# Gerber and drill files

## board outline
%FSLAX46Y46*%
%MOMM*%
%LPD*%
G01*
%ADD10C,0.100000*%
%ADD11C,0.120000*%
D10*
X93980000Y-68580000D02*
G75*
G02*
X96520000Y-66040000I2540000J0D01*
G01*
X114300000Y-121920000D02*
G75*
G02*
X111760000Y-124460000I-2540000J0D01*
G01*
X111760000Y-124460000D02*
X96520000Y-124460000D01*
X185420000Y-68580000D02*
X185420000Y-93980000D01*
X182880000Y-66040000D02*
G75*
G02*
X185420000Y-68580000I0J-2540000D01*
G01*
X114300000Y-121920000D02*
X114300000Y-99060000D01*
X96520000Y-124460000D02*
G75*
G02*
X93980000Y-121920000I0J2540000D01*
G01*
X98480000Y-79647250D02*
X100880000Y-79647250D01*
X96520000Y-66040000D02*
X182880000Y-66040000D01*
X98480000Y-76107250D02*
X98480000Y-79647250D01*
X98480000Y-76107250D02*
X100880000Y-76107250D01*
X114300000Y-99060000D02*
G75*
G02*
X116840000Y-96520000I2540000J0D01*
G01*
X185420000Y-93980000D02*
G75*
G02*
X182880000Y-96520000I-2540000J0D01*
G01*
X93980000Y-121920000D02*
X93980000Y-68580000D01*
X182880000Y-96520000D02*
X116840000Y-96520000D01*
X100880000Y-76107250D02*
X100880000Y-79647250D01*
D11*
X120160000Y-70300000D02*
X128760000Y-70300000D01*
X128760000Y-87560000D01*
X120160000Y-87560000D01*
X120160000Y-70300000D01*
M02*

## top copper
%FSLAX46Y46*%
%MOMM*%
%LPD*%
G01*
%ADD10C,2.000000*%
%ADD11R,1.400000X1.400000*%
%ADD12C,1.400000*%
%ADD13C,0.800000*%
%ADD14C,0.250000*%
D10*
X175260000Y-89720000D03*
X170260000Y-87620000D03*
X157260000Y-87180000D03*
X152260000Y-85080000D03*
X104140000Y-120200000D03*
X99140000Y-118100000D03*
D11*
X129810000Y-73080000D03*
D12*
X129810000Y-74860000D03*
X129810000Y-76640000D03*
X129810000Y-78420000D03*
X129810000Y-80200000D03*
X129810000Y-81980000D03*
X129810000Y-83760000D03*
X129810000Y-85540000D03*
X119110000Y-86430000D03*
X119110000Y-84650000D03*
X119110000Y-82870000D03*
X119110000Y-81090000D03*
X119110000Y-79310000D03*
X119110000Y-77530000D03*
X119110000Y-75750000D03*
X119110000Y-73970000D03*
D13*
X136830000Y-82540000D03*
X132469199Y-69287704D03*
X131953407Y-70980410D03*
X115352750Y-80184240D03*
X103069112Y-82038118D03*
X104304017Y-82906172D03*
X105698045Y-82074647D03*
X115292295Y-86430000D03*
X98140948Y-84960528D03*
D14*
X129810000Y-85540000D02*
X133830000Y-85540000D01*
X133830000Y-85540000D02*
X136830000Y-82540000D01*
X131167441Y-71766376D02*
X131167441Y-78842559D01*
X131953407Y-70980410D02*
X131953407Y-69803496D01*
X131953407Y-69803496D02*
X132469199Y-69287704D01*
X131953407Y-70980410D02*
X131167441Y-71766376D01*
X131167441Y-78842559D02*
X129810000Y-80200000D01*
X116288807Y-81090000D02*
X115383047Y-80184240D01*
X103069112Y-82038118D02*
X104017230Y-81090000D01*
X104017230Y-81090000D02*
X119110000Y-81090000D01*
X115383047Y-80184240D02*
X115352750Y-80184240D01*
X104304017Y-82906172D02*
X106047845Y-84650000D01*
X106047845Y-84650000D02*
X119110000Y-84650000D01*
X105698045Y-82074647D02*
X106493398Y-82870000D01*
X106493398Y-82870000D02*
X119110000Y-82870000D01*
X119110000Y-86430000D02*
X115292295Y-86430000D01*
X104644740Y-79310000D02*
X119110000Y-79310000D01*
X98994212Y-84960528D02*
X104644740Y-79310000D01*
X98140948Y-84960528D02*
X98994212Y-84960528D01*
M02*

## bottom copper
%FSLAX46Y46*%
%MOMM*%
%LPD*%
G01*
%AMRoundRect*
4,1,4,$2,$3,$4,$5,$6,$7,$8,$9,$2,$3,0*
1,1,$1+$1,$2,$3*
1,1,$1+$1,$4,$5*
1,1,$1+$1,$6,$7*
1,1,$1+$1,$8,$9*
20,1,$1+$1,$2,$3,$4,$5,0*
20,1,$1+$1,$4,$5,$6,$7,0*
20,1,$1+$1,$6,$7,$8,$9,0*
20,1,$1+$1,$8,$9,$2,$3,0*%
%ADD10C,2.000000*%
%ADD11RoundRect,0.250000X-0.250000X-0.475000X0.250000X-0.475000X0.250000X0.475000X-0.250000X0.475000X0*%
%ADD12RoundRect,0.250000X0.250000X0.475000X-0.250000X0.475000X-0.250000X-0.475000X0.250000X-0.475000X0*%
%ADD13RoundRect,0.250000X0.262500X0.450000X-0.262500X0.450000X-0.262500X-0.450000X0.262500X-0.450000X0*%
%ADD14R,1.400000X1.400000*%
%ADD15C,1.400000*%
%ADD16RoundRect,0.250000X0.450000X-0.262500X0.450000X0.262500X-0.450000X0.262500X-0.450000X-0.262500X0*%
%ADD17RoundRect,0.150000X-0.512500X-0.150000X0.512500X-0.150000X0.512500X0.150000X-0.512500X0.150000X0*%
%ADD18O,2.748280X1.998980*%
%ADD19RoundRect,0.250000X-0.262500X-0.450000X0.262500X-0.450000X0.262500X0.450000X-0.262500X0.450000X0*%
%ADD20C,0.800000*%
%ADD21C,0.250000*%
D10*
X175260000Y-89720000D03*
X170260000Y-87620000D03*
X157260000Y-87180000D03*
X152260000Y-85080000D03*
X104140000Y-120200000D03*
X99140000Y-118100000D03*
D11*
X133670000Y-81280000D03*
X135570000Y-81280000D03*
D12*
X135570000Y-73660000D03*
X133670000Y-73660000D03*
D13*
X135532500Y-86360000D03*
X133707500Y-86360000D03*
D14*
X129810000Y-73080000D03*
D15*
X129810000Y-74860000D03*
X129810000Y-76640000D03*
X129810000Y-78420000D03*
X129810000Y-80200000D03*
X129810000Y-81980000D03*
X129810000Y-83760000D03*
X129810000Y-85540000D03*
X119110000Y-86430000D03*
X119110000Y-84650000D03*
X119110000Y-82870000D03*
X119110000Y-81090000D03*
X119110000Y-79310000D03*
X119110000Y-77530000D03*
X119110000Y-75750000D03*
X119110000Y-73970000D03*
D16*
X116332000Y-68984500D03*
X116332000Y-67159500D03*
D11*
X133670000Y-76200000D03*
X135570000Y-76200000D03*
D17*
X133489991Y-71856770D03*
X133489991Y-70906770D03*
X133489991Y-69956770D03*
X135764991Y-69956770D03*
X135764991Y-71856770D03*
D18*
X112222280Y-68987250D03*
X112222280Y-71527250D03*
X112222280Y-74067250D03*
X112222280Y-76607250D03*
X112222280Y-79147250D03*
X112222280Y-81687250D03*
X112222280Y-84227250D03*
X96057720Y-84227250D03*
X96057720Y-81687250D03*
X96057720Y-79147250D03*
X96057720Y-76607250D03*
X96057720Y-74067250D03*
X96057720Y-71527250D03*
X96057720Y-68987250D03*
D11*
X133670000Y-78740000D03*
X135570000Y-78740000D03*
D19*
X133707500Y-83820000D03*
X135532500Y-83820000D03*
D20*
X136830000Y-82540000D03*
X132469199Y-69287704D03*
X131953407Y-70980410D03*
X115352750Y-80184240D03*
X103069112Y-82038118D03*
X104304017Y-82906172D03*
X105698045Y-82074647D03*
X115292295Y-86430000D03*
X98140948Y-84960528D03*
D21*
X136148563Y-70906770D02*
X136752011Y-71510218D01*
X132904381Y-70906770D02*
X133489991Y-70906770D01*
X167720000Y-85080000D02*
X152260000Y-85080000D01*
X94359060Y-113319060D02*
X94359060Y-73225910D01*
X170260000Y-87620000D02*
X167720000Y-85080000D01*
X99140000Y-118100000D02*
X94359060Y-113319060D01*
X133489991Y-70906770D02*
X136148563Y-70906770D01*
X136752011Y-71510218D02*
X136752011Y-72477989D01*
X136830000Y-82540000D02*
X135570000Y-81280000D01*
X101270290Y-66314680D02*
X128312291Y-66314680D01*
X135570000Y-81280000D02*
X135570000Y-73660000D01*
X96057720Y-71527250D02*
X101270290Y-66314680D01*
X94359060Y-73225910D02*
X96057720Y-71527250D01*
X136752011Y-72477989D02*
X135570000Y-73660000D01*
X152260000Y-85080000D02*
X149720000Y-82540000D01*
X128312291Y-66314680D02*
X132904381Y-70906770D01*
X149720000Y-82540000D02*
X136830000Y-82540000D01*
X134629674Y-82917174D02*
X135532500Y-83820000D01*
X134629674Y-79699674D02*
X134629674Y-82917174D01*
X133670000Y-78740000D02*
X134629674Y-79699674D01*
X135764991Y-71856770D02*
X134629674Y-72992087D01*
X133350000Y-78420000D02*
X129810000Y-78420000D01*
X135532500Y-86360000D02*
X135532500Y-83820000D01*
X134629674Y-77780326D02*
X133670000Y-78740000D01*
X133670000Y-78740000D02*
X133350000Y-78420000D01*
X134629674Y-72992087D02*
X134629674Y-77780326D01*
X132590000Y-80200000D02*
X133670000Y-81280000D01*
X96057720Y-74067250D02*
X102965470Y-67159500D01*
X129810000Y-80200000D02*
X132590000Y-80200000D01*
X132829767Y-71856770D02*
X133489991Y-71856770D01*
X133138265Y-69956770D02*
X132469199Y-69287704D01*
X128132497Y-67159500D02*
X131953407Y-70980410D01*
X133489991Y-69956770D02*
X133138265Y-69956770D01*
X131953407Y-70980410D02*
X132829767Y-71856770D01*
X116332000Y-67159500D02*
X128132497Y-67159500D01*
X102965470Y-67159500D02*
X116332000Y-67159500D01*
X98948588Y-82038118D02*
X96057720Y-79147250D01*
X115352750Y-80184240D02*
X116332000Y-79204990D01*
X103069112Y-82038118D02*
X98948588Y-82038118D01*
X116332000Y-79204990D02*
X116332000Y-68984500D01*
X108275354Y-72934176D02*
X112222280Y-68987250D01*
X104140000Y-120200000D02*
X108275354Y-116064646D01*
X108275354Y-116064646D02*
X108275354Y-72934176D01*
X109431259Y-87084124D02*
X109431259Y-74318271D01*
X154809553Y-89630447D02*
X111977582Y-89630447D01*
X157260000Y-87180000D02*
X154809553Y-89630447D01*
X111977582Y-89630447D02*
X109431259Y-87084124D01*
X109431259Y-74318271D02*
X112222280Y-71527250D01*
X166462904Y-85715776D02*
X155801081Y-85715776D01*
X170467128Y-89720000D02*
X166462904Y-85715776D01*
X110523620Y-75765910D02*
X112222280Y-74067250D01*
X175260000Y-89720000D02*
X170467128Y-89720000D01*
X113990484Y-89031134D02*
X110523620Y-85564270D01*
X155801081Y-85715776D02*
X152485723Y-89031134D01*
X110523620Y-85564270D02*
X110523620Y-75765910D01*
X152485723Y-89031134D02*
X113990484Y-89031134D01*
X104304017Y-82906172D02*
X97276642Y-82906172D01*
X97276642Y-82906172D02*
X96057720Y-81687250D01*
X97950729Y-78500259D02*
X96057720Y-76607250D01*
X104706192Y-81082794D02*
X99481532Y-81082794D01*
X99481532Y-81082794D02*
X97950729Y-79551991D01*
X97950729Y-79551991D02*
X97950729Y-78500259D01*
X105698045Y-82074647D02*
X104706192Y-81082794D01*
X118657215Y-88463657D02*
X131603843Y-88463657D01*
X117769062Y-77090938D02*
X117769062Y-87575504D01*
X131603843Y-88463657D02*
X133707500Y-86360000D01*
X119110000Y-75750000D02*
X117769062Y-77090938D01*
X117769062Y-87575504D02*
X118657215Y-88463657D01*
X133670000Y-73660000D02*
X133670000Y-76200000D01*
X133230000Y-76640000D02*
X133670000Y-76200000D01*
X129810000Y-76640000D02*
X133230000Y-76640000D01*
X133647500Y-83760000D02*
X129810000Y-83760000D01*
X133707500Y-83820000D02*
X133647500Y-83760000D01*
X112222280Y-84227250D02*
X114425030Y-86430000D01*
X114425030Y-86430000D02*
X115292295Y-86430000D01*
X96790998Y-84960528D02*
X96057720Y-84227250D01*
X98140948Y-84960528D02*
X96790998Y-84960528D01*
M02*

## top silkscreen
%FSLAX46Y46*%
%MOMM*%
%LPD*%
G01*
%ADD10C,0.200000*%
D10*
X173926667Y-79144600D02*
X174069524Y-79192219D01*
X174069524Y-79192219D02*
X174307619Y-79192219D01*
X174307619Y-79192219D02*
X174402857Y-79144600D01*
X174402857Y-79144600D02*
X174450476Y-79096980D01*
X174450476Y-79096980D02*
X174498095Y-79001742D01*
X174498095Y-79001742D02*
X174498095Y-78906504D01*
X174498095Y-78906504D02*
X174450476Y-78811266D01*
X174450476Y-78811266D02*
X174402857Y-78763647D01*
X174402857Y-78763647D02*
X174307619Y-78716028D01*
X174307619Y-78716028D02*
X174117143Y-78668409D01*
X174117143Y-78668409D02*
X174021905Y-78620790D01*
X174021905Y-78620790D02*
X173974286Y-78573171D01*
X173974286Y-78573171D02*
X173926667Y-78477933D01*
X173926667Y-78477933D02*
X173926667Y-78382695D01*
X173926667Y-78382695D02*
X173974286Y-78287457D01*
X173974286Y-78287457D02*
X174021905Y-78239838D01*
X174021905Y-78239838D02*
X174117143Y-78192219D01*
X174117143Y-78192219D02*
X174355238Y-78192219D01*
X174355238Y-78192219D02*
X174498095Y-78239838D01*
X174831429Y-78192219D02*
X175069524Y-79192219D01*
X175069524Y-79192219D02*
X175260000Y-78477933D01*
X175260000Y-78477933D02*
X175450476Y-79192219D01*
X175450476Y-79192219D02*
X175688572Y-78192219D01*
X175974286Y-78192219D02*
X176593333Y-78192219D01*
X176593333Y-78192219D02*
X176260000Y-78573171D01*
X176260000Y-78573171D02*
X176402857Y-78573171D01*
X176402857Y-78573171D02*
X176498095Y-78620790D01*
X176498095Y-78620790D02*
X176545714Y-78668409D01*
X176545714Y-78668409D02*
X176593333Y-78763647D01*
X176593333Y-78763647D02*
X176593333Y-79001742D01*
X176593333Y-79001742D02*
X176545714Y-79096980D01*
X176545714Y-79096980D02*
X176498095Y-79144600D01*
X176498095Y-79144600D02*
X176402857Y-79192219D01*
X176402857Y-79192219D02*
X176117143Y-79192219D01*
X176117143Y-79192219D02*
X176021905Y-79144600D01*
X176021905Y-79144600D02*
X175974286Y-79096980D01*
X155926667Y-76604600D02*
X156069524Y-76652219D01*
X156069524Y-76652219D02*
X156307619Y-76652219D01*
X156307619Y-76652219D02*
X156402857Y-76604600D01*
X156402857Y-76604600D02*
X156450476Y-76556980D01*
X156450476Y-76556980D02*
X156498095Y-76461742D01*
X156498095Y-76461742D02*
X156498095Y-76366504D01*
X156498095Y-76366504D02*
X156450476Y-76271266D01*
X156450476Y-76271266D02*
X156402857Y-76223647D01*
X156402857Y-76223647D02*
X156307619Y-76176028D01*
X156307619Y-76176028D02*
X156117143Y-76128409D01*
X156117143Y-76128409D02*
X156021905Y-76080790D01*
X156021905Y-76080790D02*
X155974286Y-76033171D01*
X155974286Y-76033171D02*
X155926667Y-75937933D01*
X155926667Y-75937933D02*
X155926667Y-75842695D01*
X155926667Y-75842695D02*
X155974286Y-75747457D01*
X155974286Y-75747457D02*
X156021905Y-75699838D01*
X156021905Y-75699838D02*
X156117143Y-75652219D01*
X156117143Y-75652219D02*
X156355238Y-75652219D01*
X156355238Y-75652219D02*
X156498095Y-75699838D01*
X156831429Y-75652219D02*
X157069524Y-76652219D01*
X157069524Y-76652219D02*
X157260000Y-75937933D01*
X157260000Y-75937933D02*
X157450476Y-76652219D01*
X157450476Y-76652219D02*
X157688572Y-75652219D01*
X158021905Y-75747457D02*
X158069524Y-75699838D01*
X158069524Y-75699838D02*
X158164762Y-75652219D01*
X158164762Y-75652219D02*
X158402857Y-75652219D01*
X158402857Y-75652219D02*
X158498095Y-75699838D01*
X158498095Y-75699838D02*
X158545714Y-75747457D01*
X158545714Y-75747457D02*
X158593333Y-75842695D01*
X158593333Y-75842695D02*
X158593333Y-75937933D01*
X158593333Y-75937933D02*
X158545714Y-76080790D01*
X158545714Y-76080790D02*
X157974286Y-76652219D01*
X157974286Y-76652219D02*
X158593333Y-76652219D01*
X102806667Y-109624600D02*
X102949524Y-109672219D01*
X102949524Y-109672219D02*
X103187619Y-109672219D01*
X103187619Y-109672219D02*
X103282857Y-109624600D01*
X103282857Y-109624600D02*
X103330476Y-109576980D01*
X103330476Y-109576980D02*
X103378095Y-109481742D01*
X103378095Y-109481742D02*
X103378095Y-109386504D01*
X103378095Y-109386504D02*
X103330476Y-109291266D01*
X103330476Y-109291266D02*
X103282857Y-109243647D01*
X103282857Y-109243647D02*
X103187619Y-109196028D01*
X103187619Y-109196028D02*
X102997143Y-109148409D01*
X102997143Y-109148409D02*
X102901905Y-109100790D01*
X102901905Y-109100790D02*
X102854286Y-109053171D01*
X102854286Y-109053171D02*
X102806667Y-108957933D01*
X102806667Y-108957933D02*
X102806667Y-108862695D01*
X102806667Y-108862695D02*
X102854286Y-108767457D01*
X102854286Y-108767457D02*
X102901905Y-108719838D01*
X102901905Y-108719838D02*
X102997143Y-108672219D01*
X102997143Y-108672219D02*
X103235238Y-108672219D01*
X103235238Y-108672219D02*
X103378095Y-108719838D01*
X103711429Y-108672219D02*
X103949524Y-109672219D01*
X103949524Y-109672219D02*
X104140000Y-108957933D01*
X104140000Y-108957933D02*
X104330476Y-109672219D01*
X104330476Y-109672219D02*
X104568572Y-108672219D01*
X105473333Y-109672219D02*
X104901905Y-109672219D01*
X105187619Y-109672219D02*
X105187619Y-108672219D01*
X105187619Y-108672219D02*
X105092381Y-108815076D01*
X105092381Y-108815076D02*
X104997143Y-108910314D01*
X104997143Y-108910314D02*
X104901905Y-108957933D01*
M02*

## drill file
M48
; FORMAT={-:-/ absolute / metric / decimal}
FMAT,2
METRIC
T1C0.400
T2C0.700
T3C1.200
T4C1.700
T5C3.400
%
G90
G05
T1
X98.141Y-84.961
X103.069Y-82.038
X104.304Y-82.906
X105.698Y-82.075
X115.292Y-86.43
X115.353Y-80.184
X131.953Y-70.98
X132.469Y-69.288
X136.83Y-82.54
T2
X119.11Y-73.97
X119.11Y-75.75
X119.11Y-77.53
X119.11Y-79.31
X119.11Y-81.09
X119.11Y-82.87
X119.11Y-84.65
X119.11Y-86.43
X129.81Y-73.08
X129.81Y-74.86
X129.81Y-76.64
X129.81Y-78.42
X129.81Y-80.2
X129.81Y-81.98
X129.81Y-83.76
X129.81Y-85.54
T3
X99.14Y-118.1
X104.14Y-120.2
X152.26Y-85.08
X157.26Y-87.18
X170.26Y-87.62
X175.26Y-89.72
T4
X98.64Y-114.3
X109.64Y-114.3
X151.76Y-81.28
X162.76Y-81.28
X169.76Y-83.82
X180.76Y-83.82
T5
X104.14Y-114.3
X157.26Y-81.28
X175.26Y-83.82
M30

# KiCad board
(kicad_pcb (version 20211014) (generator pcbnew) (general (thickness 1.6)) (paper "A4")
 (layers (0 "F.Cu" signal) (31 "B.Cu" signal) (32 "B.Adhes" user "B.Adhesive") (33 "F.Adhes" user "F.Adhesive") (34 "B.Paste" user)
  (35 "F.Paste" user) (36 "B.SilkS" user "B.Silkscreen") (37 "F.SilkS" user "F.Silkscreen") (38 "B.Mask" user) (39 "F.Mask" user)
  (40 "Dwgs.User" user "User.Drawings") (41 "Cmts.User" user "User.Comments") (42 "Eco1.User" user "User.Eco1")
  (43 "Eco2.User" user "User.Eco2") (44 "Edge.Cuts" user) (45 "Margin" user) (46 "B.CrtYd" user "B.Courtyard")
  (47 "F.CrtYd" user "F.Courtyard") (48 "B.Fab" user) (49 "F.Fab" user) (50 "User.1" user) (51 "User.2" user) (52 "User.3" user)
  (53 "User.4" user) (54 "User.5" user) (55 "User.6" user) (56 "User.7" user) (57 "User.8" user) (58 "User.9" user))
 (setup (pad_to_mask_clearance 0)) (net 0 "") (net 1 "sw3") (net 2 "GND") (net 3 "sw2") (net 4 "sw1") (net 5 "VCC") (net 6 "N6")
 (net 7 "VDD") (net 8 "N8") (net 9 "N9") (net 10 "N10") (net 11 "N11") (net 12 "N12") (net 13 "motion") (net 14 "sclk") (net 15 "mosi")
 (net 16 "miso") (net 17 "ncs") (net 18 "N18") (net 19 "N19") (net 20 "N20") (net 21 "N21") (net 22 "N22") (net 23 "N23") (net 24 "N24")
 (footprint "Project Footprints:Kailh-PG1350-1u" (layer "F.Cu") (at 175.26 83.82)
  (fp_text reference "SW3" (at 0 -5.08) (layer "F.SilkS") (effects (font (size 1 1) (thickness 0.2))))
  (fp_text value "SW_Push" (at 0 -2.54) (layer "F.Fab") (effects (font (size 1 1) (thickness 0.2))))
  (pad "" np_thru_hole circle (at 0 0 180) (size 3.4 3.4) (drill 3.4) (layers *.Cu *.Mask))
  (pad "" np_thru_hole circle (at -5.5 0 180) (size 1.7 1.7) (drill 1.7) (layers *.Cu *.Mask))
  (pad "" np_thru_hole circle (at 5.5 0 180) (size 1.7 1.7) (drill 1.7) (layers *.Cu *.Mask))
  (pad "1" thru_hole circle (at 0 5.9 180) (size 2 2) (drill 1.2) (layers *.Cu *.Mask) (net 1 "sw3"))
  (pad "2" thru_hole circle (at -5 3.8 41.9) (size 2 2) (drill 1.2) (layers *.Cu *.Mask) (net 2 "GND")))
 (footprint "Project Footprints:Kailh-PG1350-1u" (layer "F.Cu") (at 157.26 81.28)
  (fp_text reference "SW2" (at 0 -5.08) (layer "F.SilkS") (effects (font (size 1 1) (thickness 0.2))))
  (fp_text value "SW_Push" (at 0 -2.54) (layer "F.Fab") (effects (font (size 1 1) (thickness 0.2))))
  (pad "" np_thru_hole circle (at 5.5 0 180) (size 1.7 1.7) (drill 1.7) (layers *.Cu *.Mask))
  (pad "" np_thru_hole circle (at -5.5 0 180) (size 1.7 1.7) (drill 1.7) (layers *.Cu *.Mask))
  (pad "" np_thru_hole circle (at 0 0 180) (size 3.4 3.4) (drill 3.4) (layers *.Cu *.Mask))
  (pad "1" thru_hole circle (at 0 5.9 180) (size 2 2) (drill 1.2) (layers *.Cu *.Mask) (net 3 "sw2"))
  (pad "2" thru_hole circle (at -5 3.8 41.9) (size 2 2) (drill 1.2) (layers *.Cu *.Mask) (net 2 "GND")))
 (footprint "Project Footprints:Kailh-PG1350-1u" (layer "F.Cu") (at 104.14 114.3)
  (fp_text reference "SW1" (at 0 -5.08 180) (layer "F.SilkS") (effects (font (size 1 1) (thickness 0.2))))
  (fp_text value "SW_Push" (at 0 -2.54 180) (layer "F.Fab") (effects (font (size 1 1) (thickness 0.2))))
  (pad "" np_thru_hole circle (at 0 0 180) (size 3.4 3.4) (drill 3.4) (layers *.Cu *.Mask))
  (pad "" np_thru_hole circle (at 5.5 0 180) (size 1.7 1.7) (drill 1.7) (layers *.Cu *.Mask))
  (pad "" np_thru_hole circle (at -5.5 0 180) (size 1.7 1.7) (drill 1.7) (layers *.Cu *.Mask))
  (pad "1" thru_hole circle (at 0 5.9 180) (size 2 2) (drill 1.2) (layers *.Cu *.Mask) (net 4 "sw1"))
  (pad "2" thru_hole circle (at -5 3.8 41.9) (size 2 2) (drill 1.2) (layers *.Cu *.Mask) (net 2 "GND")))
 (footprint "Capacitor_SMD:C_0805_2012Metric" (layer "B.Cu") (at 134.62 81.28)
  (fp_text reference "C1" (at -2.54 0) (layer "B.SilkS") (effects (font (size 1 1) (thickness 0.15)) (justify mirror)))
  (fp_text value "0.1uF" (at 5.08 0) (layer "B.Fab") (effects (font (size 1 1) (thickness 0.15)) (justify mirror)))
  (pad "1" smd roundrect (at -0.95 0) (size 1 1.45) (layers "B.Cu" "B.Paste" "B.Mask") (roundrect_rratio 0.25) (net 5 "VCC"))
  (pad "2" smd roundrect (at 0.95 0) (size 1 1.45) (layers "B.Cu" "B.Paste" "B.Mask") (roundrect_rratio 0.25) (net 2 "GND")))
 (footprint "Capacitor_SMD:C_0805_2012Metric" (layer "B.Cu") (at 134.62 73.66 180)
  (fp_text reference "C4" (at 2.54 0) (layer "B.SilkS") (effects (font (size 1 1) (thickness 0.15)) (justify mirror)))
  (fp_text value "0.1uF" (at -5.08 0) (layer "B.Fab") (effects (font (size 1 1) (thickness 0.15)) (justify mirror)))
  (pad "1" smd roundrect (at -0.95 0 180) (size 1 1.45) (layers "B.Cu" "B.Paste" "B.Mask") (roundrect_rratio 0.25) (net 2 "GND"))
  (pad "2" smd roundrect (at 0.95 0 180) (size 1 1.45) (layers "B.Cu" "B.Paste" "B.Mask") (roundrect_rratio 0.25) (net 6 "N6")))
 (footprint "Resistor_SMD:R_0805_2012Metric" (layer "B.Cu") (at 134.62 86.36 180)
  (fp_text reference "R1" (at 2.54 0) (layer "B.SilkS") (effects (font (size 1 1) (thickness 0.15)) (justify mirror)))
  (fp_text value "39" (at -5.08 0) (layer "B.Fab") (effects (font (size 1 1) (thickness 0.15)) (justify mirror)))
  (pad "1" smd roundrect (at -0.9125 0 180) (size 1.025 1.4) (layers "B.Cu" "B.Paste" "B.Mask") (roundrect_rratio 0.243902) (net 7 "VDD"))
  (pad "2" smd roundrect (at 0.9125 0 180) (size 1.025 1.4) (layers "B.Cu" "B.Paste" "B.Mask") (roundrect_rratio 0.243902) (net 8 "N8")))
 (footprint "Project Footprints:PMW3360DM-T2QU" (layer "B.Cu") (at 124.46 78.74 -90)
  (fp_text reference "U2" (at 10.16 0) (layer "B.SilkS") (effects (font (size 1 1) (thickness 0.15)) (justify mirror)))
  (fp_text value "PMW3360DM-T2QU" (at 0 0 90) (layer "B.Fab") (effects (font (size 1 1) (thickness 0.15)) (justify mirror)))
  (fp_rect (start -8.44 4.3) (end 8.82 -4.3) (layer "Edge.Cuts") (width 0.12) (fill none))
  (pad "1" thru_hole rect (at -5.66 -5.35 270) (size 1.4 1.4) (drill 0.7) (layers *.Cu *.Mask) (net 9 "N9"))
  (pad "2" thru_hole circle (at -3.88 -5.35 270) (size 1.4 1.4) (drill 0.7) (layers *.Cu *.Mask) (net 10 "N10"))
  (pad "3" thru_hole circle (at -2.1 -5.35 270) (size 1.4 1.4) (drill 0.7) (layers *.Cu *.Mask) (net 6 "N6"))
  (pad "4" thru_hole circle (at -0.32 -5.35 270) (size 1.4 1.4) (drill 0.7) (layers *.Cu *.Mask) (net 7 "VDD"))
  (pad "5" thru_hole circle (at 1.46 -5.35 270) (size 1.4 1.4) (drill 0.7) (layers *.Cu *.Mask) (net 5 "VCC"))
  (pad "6" thru_hole circle (at 3.24 -5.35 270) (size 1.4 1.4) (drill 0.7) (layers *.Cu *.Mask) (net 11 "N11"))
  (pad "7" thru_hole circle (at 5.02 -5.35 270) (size 1.4 1.4) (drill 0.7) (layers *.Cu *.Mask) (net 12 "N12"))
  (pad "8" thru_hole circle (at 6.8 -5.35 270) (size 1.4 1.4) (drill 0.7) (layers *.Cu *.Mask) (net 2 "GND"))
  (pad "9" thru_hole circle (at 7.69 5.35 270) (size 1.4 1.4) (drill 0.7) (layers *.Cu *.Mask) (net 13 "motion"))
  (pad "10" thru_hole circle (at 5.91 5.35 270) (size 1.4 1.4) (drill 0.7) (layers *.Cu *.Mask) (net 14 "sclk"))
  (pad "11" thru_hole circle (at 4.13 5.35 270) (size 1.4 1.4) (drill 0.7) (layers *.Cu *.Mask) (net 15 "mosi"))
  (pad "12" thru_hole circle (at 2.35 5.35 270) (size 1.4 1.4) (drill 0.7) (layers *.Cu *.Mask) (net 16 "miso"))
  (pad "13" thru_hole circle (at 0.57 5.35 270) (size 1.4 1.4) (drill 0.7) (layers *.Cu *.Mask) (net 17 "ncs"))
  (pad "14" thru_hole circle (at -1.21 5.35 270) (size 1.4 1.4) (drill 0.7) (layers *.Cu *.Mask) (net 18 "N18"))
  (pad "15" thru_hole circle (at -2.99 5.35 270) (size 1.4 1.4) (drill 0.7) (layers *.Cu *.Mask) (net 8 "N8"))
  (pad "16" thru_hole circle (at -4.77 5.35 270) (size 1.4 1.4) (drill 0.7) (layers *.Cu *.Mask) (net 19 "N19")))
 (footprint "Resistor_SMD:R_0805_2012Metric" (layer "B.Cu") (at 116.332 68.072 90)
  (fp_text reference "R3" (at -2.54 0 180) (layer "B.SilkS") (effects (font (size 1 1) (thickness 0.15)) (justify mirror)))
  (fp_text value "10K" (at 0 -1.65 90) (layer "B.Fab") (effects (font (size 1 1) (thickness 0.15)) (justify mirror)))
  (pad "1" smd roundrect (at -0.9125 0 90) (size 1.025 1.4) (layers "B.Cu" "B.Paste" "B.Mask") (roundrect_rratio 0.243902) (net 16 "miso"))
  (pad "2" smd roundrect (at 0.9125 0 90) (size 1.025 1.4) (layers "B.Cu" "B.Paste" "B.Mask") (roundrect_rratio 0.243902) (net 5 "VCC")))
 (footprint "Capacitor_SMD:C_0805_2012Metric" (layer "B.Cu") (at 134.62 76.2)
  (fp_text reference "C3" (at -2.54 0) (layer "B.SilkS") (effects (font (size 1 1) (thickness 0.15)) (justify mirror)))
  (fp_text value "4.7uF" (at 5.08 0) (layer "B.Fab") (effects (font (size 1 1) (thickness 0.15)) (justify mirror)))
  (pad "1" smd roundrect (at -0.95 0) (size 1 1.45) (layers "B.Cu" "B.Paste" "B.Mask") (roundrect_rratio 0.25) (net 6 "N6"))
  (pad "2" smd roundrect (at 0.95 0) (size 1 1.45) (layers "B.Cu" "B.Paste" "B.Mask") (roundrect_rratio 0.25) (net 2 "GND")))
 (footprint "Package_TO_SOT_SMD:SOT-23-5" (layer "B.Cu") (at 134.627491 70.90677)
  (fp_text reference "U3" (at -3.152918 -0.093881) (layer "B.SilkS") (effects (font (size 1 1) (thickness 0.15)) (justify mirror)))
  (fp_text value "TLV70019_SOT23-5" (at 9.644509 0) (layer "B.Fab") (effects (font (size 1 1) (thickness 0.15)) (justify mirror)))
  (pad "1" smd roundrect (at -1.1375 0.95) (size 1.325 0.6) (layers "B.Cu" "B.Paste" "B.Mask") (roundrect_rratio 0.25) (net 5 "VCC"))
  (pad "2" smd roundrect (at -1.1375 0) (size 1.325 0.6) (layers "B.Cu" "B.Paste" "B.Mask") (roundrect_rratio 0.25) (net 2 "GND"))
  (pad "3" smd roundrect (at -1.1375 -0.95) (size 1.325 0.6) (layers "B.Cu" "B.Paste" "B.Mask") (roundrect_rratio 0.25) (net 5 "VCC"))
  (pad "4" smd roundrect (at 1.1375 -0.95) (size 1.325 0.6) (layers "B.Cu" "B.Paste" "B.Mask") (roundrect_rratio 0.25) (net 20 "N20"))
  (pad "5" smd roundrect (at 1.1375 0.95) (size 1.325 0.6) (layers "B.Cu" "B.Paste" "B.Mask") (roundrect_rratio 0.25) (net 7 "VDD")))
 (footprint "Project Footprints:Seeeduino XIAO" (layer "B.Cu") (at 104.14 76.60725 180)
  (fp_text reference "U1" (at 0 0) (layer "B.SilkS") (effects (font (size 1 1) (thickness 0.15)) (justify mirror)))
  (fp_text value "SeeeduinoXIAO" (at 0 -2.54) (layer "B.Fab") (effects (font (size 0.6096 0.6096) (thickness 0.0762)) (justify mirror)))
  (pad "1" smd oval (at -8.08228 7.62 180) (size 2.74828 1.99898) (layers "B.Cu" "B.Paste" "B.Mask") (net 4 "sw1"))
  (pad "2" smd oval (at -8.08228 5.08 180) (size 2.74828 1.99898) (layers "B.Cu" "B.Paste" "B.Mask") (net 3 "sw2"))
  (pad "3" smd oval (at -8.08228 2.54 180) (size 2.74828 1.99898) (layers "B.Cu" "B.Paste" "B.Mask") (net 1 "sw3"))
  (pad "4" smd oval (at -8.08228 0 180) (size 2.74828 1.99898) (layers "B.Cu" "B.Paste" "B.Mask") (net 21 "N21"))
  (pad "5" smd oval (at -8.08228 -2.54 180) (size 2.74828 1.99898) (layers "B.Cu" "B.Paste" "B.Mask") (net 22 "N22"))
  (pad "6" smd oval (at -8.08228 -5.08 180) (size 2.74828 1.99898) (layers "B.Cu" "B.Paste" "B.Mask") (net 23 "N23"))
  (pad "7" smd oval (at -8.08228 -7.62 180) (size 2.74828 1.99898) (layers "B.Cu" "B.Paste" "B.Mask") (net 13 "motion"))
  (pad "8" smd oval (at 8.08228 -7.62 180) (size 2.74828 1.99898) (layers "B.Cu" "B.Paste" "B.Mask") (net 17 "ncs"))
  (pad "9" smd oval (at 8.08228 -5.08 180) (size 2.74828 1.99898) (layers "B.Cu" "B.Paste" "B.Mask") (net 14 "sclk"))
  (pad "10" smd oval (at 8.08228 -2.54 180) (size 2.74828 1.99898) (layers "B.Cu" "B.Paste" "B.Mask") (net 16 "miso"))
  (pad "11" smd oval (at 8.08228 0 180) (size 2.74828 1.99898) (layers "B.Cu" "B.Paste" "B.Mask") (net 15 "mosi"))
  (pad "12" smd oval (at 8.08228 2.54 180) (size 2.74828 1.99898) (layers "B.Cu" "B.Paste" "B.Mask") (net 5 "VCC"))
  (pad "13" smd oval (at 8.08228 5.08 180) (size 2.74828 1.99898) (layers "B.Cu" "B.Paste" "B.Mask") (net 2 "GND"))
  (pad "14" smd oval (at 8.08228 7.62 180) (size 2.74828 1.99898) (layers "B.Cu" "B.Paste" "B.Mask") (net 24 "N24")))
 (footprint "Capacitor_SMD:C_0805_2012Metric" (layer "B.Cu") (at 134.62 78.74)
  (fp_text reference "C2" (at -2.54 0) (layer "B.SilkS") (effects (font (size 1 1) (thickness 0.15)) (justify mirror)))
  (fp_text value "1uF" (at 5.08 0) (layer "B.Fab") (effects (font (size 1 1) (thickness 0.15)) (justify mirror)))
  (pad "1" smd roundrect (at -0.95 0) (size 1 1.45) (layers "B.Cu" "B.Paste" "B.Mask") (roundrect_rratio 0.25) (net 7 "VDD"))
  (pad "2" smd roundrect (at 0.95 0) (size 1 1.45) (layers "B.Cu" "B.Paste" "B.Mask") (roundrect_rratio 0.25) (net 2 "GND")))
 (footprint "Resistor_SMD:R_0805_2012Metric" (layer "B.Cu") (at 134.62 83.82)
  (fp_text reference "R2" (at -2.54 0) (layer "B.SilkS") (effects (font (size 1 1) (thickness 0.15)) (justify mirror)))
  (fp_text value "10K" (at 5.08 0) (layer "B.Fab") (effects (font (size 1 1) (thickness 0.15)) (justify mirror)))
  (pad "1" smd roundrect (at -0.9125 0) (size 1.025 1.4) (layers "B.Cu" "B.Paste" "B.Mask") (roundrect_rratio 0.243902) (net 12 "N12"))
  (pad "2" smd roundrect (at 0.9125 0) (size 1.025 1.4) (layers "B.Cu" "B.Paste" "B.Mask") (roundrect_rratio 0.243902) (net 7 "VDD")))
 (gr_arc (start 93.98 68.58) (mid 94.723949 66.783949) (end 96.52 66.04) (layer "Edge.Cuts") (width 0.1))
 (gr_arc (start 114.3 121.92) (mid 113.556051 123.716051) (end 111.76 124.46) (layer "Edge.Cuts") (width 0.1))
 (gr_line (start 111.76 124.46) (end 96.52 124.46) (layer "Edge.Cuts") (width 0.1))
 (gr_line (start 185.42 68.58) (end 185.42 93.98) (layer "Edge.Cuts") (width 0.1))
 (gr_arc (start 182.88 66.04) (mid 184.676051 66.783949) (end 185.42 68.58) (layer "Edge.Cuts") (width 0.1))
 (gr_line (start 114.3 121.92) (end 114.3 99.06) (layer "Edge.Cuts") (width 0.1))
 (gr_arc (start 96.52 124.46) (mid 94.723949 123.716051) (end 93.98 121.92) (layer "Edge.Cuts") (width 0.1))
 (gr_line (start 98.48 79.64725) (end 100.88 79.64725) (layer "Edge.Cuts") (width 0.1))
 (gr_line (start 96.52 66.04) (end 182.88 66.04) (layer "Edge.Cuts") (width 0.1))
 (gr_line (start 98.48 76.10725) (end 98.48 79.64725) (layer "Edge.Cuts") (width 0.1))
 (gr_line (start 98.48 76.10725) (end 100.88 76.10725) (layer "Edge.Cuts") (width 0.1))
 (gr_arc (start 114.3 99.06) (mid 115.043949 97.263949) (end 116.84 96.52) (layer "Edge.Cuts") (width 0.1))
 (gr_arc (start 185.42 93.98) (mid 184.676051 95.776051) (end 182.88 96.52) (layer "Edge.Cuts") (width 0.1))
 (gr_line (start 93.98 121.92) (end 93.98 68.58) (layer "Edge.Cuts") (width 0.1))
 (gr_line (start 182.88 96.52) (end 116.84 96.52) (layer "Edge.Cuts") (width 0.1))
 (gr_line (start 100.88 76.10725) (end 100.88 79.64725) (layer "Edge.Cuts") (width 0.1))
 (segment (start 129.81 85.54) (end 133.83 85.54) (width 0.25) (layer "F.Cu") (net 2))
 (segment (start 133.83 85.54) (end 136.83 82.54) (width 0.25) (layer "F.Cu") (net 2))
 (via (at 136.83 82.54) (size 0.8) (drill 0.4) (layers "F.Cu" "B.Cu") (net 2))
 (segment (start 136.148563 70.90677) (end 136.752011 71.510218) (width 0.25) (layer "B.Cu") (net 2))
 (segment (start 132.904381 70.90677) (end 133.489991 70.90677) (width 0.25) (layer "B.Cu") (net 2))
 (segment (start 167.72 85.08) (end 152.26 85.08) (width 0.25) (layer "B.Cu") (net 2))
 (segment (start 94.35906 113.31906) (end 94.35906 73.22591) (width 0.25) (layer "B.Cu") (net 2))
 (segment (start 170.26 87.62) (end 167.72 85.08) (width 0.25) (layer "B.Cu") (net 2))
 (segment (start 99.14 118.1) (end 94.35906 113.31906) (width 0.25) (layer "B.Cu") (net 2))
 (segment (start 133.489991 70.90677) (end 136.148563 70.90677) (width 0.25) (layer "B.Cu") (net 2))
 (segment (start 136.752011 71.510218) (end 136.752011 72.477989) (width 0.25) (layer "B.Cu") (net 2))
 (segment (start 136.83 82.54) (end 135.57 81.28) (width 0.25) (layer "B.Cu") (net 2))
 (segment (start 101.27029 66.31468) (end 128.312291 66.31468) (width 0.25) (layer "B.Cu") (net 2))
 (segment (start 135.57 81.28) (end 135.57 73.66) (width 0.25) (layer "B.Cu") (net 2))
 (segment (start 96.05772 71.52725) (end 101.27029 66.31468) (width 0.25) (layer "B.Cu") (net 2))
 (segment (start 94.35906 73.22591) (end 96.05772 71.52725) (width 0.25) (layer "B.Cu") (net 2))
 (segment (start 136.752011 72.477989) (end 135.57 73.66) (width 0.25) (layer "B.Cu") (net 2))
 (segment (start 152.26 85.08) (end 149.72 82.54) (width 0.25) (layer "B.Cu") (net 2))
 (segment (start 128.312291 66.31468) (end 132.904381 70.90677) (width 0.25) (layer "B.Cu") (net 2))
 (segment (start 149.72 82.54) (end 136.83 82.54) (width 0.25) (layer "B.Cu") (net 2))
 (segment (start 134.629674 82.917174) (end 135.5325 83.82) (width 0.25) (layer "B.Cu") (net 7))
 (segment (start 134.629674 79.699674) (end 134.629674 82.917174) (width 0.25) (layer "B.Cu") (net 7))
 (segment (start 133.67 78.74) (end 134.629674 79.699674) (width 0.25) (layer "B.Cu") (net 7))
 (segment (start 135.764991 71.85677) (end 134.629674 72.992087) (width 0.25) (layer "B.Cu") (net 7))
 (segment (start 133.35 78.42) (end 129.81 78.42) (width 0.25) (layer "B.Cu") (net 7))
 (segment (start 135.5325 86.36) (end 135.5325 83.82) (width 0.25) (layer "B.Cu") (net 7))
 (segment (start 134.629674 77.780326) (end 133.67 78.74) (width 0.25) (layer "B.Cu") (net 7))
 (segment (start 133.67 78.74) (end 133.35 78.42) (width 0.25) (layer "B.Cu") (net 7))
 (segment (start 134.629674 72.992087) (end 134.629674 77.780326) (width 0.25) (layer "B.Cu") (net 7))
 (segment (start 131.167441 71.766376) (end 131.167441 78.842559) (width 0.25) (layer "F.Cu") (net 5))
 (segment (start 131.953407 70.98041) (end 131.953407 69.803496) (width 0.25) (layer "F.Cu") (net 5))
 (segment (start 131.953407 69.803496) (end 132.469199 69.287704) (width 0.25) (layer "F.Cu") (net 5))
 (segment (start 131.953407 70.98041) (end 131.167441 71.766376) (width 0.25) (layer "F.Cu") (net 5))
 (segment (start 131.167441 78.842559) (end 129.81 80.2) (width 0.25) (layer "F.Cu") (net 5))
 (via (at 132.469199 69.287704) (size 0.8) (drill 0.4) (layers "F.Cu" "B.Cu") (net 5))
 (via (at 131.953407 70.98041) (size 0.8) (drill 0.4) (layers "F.Cu" "B.Cu") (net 5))
 (segment (start 132.59 80.2) (end 133.67 81.28) (width 0.25) (layer "B.Cu") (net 5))
 (segment (start 96.05772 74.06725) (end 102.96547 67.1595) (width 0.25) (layer "B.Cu") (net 5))
 (segment (start 129.81 80.2) (end 132.59 80.2) (width 0.25) (layer "B.Cu") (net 5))
 (segment (start 132.829767 71.85677) (end 133.489991 71.85677) (width 0.25) (layer "B.Cu") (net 5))
 (segment (start 133.138265 69.95677) (end 132.469199 69.287704) (width 0.25) (layer "B.Cu") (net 5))
 (segment (start 128.132497 67.1595) (end 131.953407 70.98041) (width 0.25) (layer "B.Cu") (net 5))
 (segment (start 133.489991 69.95677) (end 133.138265 69.95677) (width 0.25) (layer "B.Cu") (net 5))
 (segment (start 131.953407 70.98041) (end 132.829767 71.85677) (width 0.25) (layer "B.Cu") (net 5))
 (segment (start 116.332 67.1595) (end 128.132497 67.1595) (width 0.25) (layer "B.Cu") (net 5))
 (segment (start 102.96547 67.1595) (end 116.332 67.1595) (width 0.25) (layer "B.Cu") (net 5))
 (segment (start 116.288807 81.09) (end 115.383047 80.18424) (width 0.25) (layer "F.Cu") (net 16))
 (segment (start 103.069112 82.038118) (end 104.01723 81.09) (width 0.25) (layer "F.Cu") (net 16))
 (segment (start 104.01723 81.09) (end 119.11 81.09) (width 0.25) (layer "F.Cu") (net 16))
 (segment (start 115.383047 80.18424) (end 115.35275 80.18424) (width 0.25) (layer "F.Cu") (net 16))
 (via (at 115.35275 80.18424) (size 0.8) (drill 0.4) (layers "F.Cu" "B.Cu") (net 16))
 (via (at 103.069112 82.038118) (size 0.8) (drill 0.4) (layers "F.Cu" "B.Cu") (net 16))
 (segment (start 98.948588 82.038118) (end 96.05772 79.14725) (width 0.25) (layer "B.Cu") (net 16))
 (segment (start 115.35275 80.18424) (end 116.332 79.20499) (width 0.25) (layer "B.Cu") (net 16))
 (segment (start 103.069112 82.038118) (end 98.948588 82.038118) (width 0.25) (layer "B.Cu") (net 16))
 (segment (start 116.332 79.20499) (end 116.332 68.9845) (width 0.25) (layer "B.Cu") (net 16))
 (segment (start 108.275354 72.934176) (end 112.22228 68.98725) (width 0.25) (layer "B.Cu") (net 4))
 (segment (start 104.14 120.2) (end 108.275354 116.064646) (width 0.25) (layer "B.Cu") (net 4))
 (segment (start 108.275354 116.064646) (end 108.275354 72.934176) (width 0.25) (layer "B.Cu") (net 4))
 (segment (start 109.431259 87.084124) (end 109.431259 74.318271) (width 0.25) (layer "B.Cu") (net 3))
 (segment (start 154.809553 89.630447) (end 111.977582 89.630447) (width 0.25) (layer "B.Cu") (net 3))
 (segment (start 157.26 87.18) (end 154.809553 89.630447) (width 0.25) (layer "B.Cu") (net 3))
 (segment (start 111.977582 89.630447) (end 109.431259 87.084124) (width 0.25) (layer "B.Cu") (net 3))
 (segment (start 109.431259 74.318271) (end 112.22228 71.52725) (width 0.25) (layer "B.Cu") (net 3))
 (segment (start 166.462904 85.715776) (end 155.801081 85.715776) (width 0.25) (layer "B.Cu") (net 1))
 (segment (start 170.467128 89.72) (end 166.462904 85.715776) (width 0.25) (layer "B.Cu") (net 1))
 (segment (start 110.52362 75.76591) (end 112.22228 74.06725) (width 0.25) (layer "B.Cu") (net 1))
 (segment (start 175.26 89.72) (end 170.467128 89.72) (width 0.25) (layer "B.Cu") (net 1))
 (segment (start 113.990484 89.031134) (end 110.52362 85.56427) (width 0.25) (layer "B.Cu") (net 1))
 (segment (start 155.801081 85.715776) (end 152.485723 89.031134) (width 0.25) (layer "B.Cu") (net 1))
 (segment (start 110.52362 85.56427) (end 110.52362 75.76591) (width 0.25) (layer "B.Cu") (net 1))
 (segment (start 152.485723 89.031134) (end 113.990484 89.031134) (width 0.25) (layer "B.Cu") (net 1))
 (segment (start 104.304017 82.906172) (end 106.047845 84.65) (width 0.25) (layer "F.Cu") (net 14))
 (segment (start 106.047845 84.65) (end 119.11 84.65) (width 0.25) (layer "F.Cu") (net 14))
 (via (at 104.304017 82.906172) (size 0.8) (drill 0.4) (layers "F.Cu" "B.Cu") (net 14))
 (segment (start 104.304017 82.906172) (end 97.276642 82.906172) (width 0.25) (layer "B.Cu") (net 14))
 (segment (start 97.276642 82.906172) (end 96.05772 81.68725) (width 0.25) (layer "B.Cu") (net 14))
 (segment (start 105.698045 82.074647) (end 106.493398 82.87) (width 0.25) (layer "F.Cu") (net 15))
 (segment (start 106.493398 82.87) (end 119.11 82.87) (width 0.25) (layer "F.Cu") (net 15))
 (via (at 105.698045 82.074647) (size 0.8) (drill 0.4) (layers "F.Cu" "B.Cu") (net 15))
 (segment (start 97.950729 78.500259) (end 96.05772 76.60725) (width 0.25) (layer "B.Cu") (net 15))
 (segment (start 104.706192 81.082794) (end 99.481532 81.082794) (width 0.25) (layer "B.Cu") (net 15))
 (segment (start 99.481532 81.082794) (end 97.950729 79.551991) (width 0.25) (layer "B.Cu") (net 15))
 (segment (start 97.950729 79.551991) (end 97.950729 78.500259) (width 0.25) (layer "B.Cu") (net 15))
 (segment (start 105.698045 82.074647) (end 104.706192 81.082794) (width 0.25) (layer "B.Cu") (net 15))
 (segment (start 118.657215 88.463657) (end 131.603843 88.463657) (width 0.25) (layer "B.Cu") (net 8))
 (segment (start 117.769062 77.090938) (end 117.769062 87.575504) (width 0.25) (layer "B.Cu") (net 8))
 (segment (start 131.603843 88.463657) (end 133.7075 86.36) (width 0.25) (layer "B.Cu") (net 8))
 (segment (start 119.11 75.75) (end 117.769062 77.090938) (width 0.25) (layer "B.Cu") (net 8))
 (segment (start 117.769062 87.575504) (end 118.657215 88.463657) (width 0.25) (layer "B.Cu") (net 8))
 (segment (start 133.67 73.66) (end 133.67 76.2) (width 0.25) (layer "B.Cu") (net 6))
 (segment (start 133.23 76.64) (end 133.67 76.2) (width 0.25) (layer "B.Cu") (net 6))
 (segment (start 129.81 76.64) (end 133.23 76.64) (width 0.25) (layer "B.Cu") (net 6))
 (segment (start 133.6475 83.76) (end 129.81 83.76) (width 0.25) (layer "B.Cu") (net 12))
 (segment (start 133.7075 83.82) (end 133.6475 83.76) (width 0.25) (layer "B.Cu") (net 12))
 (segment (start 119.11 86.43) (end 115.292295 86.43) (width 0.25) (layer "F.Cu") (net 13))
 (via (at 115.292295 86.43) (size 0.8) (drill 0.4) (layers "F.Cu" "B.Cu") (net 13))
 (segment (start 112.22228 84.22725) (end 114.42503 86.43) (width 0.25) (layer "B.Cu") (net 13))
 (segment (start 114.42503 86.43) (end 115.292295 86.43) (width 0.25) (layer "B.Cu") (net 13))
 (segment (start 104.64474 79.31) (end 119.11 79.31) (width 0.25) (layer "F.Cu") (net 17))
 (segment (start 98.994212 84.960528) (end 104.64474 79.31) (width 0.25) (layer "F.Cu") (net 17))
 (segment (start 98.140948 84.960528) (end 98.994212 84.960528) (width 0.25) (layer "F.Cu") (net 17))
 (via (at 98.140948 84.960528) (size 0.8) (drill 0.4) (layers "F.Cu" "B.Cu") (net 17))
 (segment (start 96.790998 84.960528) (end 96.05772 84.22725) (width 0.25) (layer "B.Cu") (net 17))
 (segment (start 98.140948 84.960528) (end 96.790998 84.960528) (width 0.25) (layer "B.Cu") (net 17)))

